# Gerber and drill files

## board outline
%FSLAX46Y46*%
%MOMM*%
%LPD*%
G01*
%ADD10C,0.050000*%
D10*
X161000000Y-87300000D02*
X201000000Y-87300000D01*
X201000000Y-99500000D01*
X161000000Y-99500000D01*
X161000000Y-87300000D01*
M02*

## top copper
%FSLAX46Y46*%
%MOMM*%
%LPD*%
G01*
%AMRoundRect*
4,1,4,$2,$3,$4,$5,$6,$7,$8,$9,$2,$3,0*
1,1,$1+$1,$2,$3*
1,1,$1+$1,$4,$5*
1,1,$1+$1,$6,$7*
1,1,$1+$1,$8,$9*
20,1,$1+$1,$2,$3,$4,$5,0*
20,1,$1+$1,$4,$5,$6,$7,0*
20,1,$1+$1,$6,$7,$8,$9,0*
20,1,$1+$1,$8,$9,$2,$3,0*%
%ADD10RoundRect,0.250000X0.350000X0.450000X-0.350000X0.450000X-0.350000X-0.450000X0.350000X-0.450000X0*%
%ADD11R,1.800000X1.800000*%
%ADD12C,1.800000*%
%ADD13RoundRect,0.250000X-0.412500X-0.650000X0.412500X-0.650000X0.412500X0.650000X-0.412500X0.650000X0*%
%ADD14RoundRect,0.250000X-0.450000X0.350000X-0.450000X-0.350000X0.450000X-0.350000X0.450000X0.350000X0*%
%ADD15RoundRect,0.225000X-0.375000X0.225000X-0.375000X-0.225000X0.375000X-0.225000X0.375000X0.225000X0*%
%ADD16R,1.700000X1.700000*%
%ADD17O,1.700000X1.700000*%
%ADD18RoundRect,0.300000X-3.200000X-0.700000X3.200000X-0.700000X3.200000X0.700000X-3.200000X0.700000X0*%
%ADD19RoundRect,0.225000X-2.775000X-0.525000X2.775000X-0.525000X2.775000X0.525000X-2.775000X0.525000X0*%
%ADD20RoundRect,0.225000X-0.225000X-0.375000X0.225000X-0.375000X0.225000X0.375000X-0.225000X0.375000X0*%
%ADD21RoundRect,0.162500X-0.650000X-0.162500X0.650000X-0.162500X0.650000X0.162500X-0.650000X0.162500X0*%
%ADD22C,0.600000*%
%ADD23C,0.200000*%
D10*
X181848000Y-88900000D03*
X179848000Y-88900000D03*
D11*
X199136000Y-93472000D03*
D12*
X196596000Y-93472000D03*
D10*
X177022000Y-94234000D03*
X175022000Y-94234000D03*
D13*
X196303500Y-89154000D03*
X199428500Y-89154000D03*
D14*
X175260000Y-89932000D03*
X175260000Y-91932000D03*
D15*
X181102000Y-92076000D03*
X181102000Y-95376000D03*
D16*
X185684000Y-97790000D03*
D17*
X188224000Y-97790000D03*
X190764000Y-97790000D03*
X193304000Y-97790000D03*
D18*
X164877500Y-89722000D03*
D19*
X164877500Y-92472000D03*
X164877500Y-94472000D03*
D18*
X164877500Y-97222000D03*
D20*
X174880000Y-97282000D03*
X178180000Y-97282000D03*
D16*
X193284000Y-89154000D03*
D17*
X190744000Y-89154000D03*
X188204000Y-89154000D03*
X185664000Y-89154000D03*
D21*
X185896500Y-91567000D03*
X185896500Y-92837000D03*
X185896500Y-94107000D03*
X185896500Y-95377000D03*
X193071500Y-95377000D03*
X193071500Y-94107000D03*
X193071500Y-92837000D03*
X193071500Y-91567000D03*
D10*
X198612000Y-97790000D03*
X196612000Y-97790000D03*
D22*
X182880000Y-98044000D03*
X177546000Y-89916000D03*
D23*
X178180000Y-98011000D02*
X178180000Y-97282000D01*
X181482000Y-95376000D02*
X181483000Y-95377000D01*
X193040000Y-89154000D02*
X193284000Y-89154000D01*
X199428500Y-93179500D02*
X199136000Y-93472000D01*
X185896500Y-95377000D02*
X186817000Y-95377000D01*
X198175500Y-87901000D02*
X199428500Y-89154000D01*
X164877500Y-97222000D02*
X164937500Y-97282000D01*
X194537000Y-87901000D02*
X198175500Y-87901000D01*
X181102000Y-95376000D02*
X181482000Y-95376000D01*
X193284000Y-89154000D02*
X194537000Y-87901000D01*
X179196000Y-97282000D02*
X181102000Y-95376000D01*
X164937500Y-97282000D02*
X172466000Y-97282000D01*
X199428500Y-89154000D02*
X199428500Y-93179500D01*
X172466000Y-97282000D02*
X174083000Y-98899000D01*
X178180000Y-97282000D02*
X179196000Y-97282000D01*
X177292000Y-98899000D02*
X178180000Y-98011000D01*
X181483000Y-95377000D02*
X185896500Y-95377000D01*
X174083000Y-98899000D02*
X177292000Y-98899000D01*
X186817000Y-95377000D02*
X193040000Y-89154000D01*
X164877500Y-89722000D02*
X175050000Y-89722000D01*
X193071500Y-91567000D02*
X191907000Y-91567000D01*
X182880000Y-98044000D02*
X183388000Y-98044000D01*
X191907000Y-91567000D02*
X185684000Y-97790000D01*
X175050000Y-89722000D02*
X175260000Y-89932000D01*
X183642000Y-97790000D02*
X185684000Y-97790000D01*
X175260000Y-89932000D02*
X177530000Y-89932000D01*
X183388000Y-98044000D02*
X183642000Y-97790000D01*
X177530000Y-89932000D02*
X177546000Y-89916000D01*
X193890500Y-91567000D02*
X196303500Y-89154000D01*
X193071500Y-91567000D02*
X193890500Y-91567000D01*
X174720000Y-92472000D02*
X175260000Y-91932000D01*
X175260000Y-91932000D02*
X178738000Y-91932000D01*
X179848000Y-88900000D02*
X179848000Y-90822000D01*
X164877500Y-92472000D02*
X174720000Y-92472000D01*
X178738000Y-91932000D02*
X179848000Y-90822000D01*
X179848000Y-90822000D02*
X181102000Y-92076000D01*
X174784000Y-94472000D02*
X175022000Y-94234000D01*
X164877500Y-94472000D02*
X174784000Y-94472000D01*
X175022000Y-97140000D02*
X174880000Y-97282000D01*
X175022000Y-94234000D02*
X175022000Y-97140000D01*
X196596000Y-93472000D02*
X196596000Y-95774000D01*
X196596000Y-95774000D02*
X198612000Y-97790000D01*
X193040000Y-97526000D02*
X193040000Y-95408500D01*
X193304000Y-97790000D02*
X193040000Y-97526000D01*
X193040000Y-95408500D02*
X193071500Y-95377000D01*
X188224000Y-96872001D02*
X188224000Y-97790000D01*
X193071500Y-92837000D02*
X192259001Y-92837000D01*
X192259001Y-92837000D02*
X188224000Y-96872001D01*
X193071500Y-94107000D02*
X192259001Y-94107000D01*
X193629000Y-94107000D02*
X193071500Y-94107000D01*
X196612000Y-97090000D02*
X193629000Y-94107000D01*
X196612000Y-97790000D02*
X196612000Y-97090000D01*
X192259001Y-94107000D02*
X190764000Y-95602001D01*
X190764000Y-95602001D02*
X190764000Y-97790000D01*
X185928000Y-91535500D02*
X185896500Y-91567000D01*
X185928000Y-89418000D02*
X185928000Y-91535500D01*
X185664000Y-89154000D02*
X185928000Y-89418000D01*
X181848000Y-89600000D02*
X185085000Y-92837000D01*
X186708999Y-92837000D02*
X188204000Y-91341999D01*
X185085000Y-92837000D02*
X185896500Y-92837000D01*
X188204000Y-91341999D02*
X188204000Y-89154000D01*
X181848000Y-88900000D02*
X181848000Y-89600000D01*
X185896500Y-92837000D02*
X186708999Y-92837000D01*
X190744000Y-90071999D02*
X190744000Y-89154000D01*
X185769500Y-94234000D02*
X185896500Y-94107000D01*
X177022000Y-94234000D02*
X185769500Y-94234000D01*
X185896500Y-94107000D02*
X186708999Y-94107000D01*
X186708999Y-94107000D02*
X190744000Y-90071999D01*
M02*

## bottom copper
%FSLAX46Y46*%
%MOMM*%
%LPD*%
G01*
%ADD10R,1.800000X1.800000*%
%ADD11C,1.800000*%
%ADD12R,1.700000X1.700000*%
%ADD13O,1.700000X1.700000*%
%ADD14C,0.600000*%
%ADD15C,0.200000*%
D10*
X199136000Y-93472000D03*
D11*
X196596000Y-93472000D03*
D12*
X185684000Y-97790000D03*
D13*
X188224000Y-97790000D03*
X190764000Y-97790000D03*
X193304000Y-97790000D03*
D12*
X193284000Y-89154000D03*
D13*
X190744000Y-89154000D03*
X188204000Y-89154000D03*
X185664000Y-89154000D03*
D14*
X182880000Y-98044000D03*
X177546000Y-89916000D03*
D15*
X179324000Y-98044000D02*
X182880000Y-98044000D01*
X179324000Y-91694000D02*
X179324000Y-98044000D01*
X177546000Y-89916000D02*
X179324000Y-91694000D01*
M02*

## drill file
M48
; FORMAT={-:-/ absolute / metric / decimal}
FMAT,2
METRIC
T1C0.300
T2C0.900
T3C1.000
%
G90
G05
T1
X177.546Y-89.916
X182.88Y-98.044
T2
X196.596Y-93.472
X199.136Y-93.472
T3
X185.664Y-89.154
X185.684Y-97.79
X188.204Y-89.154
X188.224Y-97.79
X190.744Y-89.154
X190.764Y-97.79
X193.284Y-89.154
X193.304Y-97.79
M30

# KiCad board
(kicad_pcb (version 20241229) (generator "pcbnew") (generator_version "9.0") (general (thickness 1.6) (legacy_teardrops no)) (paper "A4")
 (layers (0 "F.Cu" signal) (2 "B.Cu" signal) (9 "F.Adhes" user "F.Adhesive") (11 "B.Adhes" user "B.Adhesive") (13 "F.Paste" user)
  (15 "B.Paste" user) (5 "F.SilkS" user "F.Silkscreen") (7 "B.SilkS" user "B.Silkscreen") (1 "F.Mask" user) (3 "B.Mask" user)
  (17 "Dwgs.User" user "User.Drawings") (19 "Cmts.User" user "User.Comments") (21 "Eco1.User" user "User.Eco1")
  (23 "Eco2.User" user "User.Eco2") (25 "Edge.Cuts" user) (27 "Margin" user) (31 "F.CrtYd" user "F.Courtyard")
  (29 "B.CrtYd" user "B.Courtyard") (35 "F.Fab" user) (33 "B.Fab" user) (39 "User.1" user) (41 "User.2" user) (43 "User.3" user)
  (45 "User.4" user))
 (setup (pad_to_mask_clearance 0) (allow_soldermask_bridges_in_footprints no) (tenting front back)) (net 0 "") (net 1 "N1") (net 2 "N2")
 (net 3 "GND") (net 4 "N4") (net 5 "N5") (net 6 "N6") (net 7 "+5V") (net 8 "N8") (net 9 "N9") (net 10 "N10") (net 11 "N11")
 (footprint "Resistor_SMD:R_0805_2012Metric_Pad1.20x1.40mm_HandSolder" (layer "F.Cu") (at 180.848 88.9 180)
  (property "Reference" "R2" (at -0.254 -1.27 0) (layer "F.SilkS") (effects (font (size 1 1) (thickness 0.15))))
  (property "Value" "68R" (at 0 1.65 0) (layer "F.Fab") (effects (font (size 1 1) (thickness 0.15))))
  (pad "1" smd roundrect (at -1 0 180) (size 1.2 1.4) (layers "F.Cu" "F.Mask" "F.Paste") (roundrect_rratio 0.208333) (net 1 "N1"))
  (pad "2" smd roundrect (at 1 0 180) (size 1.2 1.4) (layers "F.Cu" "F.Mask" "F.Paste") (roundrect_rratio 0.208333) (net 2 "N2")))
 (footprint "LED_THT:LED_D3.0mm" (layer "F.Cu") (at 199.136 93.472 180)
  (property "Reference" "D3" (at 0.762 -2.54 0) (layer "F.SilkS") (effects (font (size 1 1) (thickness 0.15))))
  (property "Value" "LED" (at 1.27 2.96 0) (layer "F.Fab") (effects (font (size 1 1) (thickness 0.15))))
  (pad "1" thru_hole rect (at 0 0 180) (size 1.8 1.8) (drill 0.9) (layers "*.Cu" "*.Mask") (remove_unused_layers no) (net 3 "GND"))
  (pad "2" thru_hole circle (at 2.54 0 180) (size 1.8 1.8) (drill 0.9) (layers "*.Cu" "*.Mask") (remove_unused_layers no) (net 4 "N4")))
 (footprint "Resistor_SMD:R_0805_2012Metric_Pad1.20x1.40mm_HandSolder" (layer "F.Cu") (at 176.022 94.234 180)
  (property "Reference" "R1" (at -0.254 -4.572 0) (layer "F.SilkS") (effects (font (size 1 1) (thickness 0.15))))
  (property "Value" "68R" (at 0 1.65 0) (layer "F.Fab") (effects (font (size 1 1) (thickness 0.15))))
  (pad "1" smd roundrect (at -1 0 180) (size 1.2 1.4) (layers "F.Cu" "F.Mask" "F.Paste") (roundrect_rratio 0.208333) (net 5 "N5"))
  (pad "2" smd roundrect (at 1 0 180) (size 1.2 1.4) (layers "F.Cu" "F.Mask" "F.Paste") (roundrect_rratio 0.208333) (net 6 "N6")))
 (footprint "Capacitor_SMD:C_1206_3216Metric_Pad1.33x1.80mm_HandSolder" (layer "F.Cu") (at 197.866 89.154)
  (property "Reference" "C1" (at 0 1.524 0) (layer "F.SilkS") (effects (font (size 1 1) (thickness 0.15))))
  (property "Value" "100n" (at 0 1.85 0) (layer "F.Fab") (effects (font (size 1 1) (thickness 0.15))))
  (pad "1" smd roundrect (at -1.5625 0) (size 1.325 1.8) (layers "F.Cu" "F.Mask" "F.Paste") (roundrect_rratio 0.188679) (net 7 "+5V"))
  (pad "2" smd roundrect (at 1.5625 0) (size 1.325 1.8) (layers "F.Cu" "F.Mask" "F.Paste") (roundrect_rratio 0.188679) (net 3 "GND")))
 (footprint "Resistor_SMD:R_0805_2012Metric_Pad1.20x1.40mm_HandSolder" (layer "F.Cu") (at 175.26 90.932 -90)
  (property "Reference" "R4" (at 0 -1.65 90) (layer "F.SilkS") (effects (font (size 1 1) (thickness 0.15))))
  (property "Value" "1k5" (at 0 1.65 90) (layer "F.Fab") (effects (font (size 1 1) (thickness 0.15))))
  (pad "1" smd roundrect (at -1 0 270) (size 1.2 1.4) (layers "F.Cu" "F.Mask" "F.Paste") (roundrect_rratio 0.208333) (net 7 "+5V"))
  (pad "2" smd roundrect (at 1 0 270) (size 1.2 1.4) (layers "F.Cu" "F.Mask" "F.Paste") (roundrect_rratio 0.208333) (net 2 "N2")))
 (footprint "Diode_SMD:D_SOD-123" (layer "F.Cu") (at 181.102 93.726 -90)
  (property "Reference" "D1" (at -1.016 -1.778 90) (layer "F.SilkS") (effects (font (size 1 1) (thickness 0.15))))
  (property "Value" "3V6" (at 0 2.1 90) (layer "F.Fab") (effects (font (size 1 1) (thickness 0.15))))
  (pad "1" smd roundrect (at -1.65 0 270) (size 0.9 1.2) (layers "F.Cu" "F.Mask" "F.Paste") (roundrect_rratio 0.25) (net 2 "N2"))
  (pad "2" smd roundrect (at 1.65 0 270) (size 0.9 1.2) (layers "F.Cu" "F.Mask" "F.Paste") (roundrect_rratio 0.25) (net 3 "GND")))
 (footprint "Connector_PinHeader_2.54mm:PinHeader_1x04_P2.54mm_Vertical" (layer "F.Cu") (at 185.684 97.79 90)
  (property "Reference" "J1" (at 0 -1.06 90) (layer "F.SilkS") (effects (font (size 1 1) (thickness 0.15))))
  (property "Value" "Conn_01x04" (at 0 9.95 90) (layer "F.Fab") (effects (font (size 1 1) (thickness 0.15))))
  (pad "1" thru_hole rect (at 0 0 90) (size 1.7 1.7) (drill 1) (layers "*.Cu" "*.Mask") (remove_unused_layers no) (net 7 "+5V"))
  (pad "2" thru_hole oval (at 0 2.54 90) (size 1.7 1.7) (drill 1) (layers "*.Cu" "*.Mask") (remove_unused_layers no) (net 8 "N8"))
  (pad "3" thru_hole oval (at 0 5.08 90) (size 1.7 1.7) (drill 1) (layers "*.Cu" "*.Mask") (remove_unused_layers no) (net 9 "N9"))
  (pad "4" thru_hole oval (at 0 7.62 90) (size 1.7 1.7) (drill 1) (layers "*.Cu" "*.Mask") (remove_unused_layers no) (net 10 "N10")))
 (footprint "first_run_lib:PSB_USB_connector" (layer "F.Cu") (at 164.8775 93.472)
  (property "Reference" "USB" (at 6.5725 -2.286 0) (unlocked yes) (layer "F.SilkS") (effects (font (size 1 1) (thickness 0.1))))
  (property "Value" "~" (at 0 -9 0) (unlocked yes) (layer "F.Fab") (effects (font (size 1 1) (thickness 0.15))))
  (pad "1" smd roundrect (at 0 -3.75) (size 7 2) (layers "F.Cu" "F.Mask" "F.Paste") (roundrect_rratio 0.15) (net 7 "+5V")
   (thermal_bridge_angle 45))
  (pad "2" smd roundrect (at 0 -1) (size 6 1.5) (layers "F.Cu" "F.Mask" "F.Paste") (roundrect_rratio 0.15) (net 2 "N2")
   (thermal_bridge_angle 45))
  (pad "3" smd roundrect (at 0 1) (size 6 1.5) (layers "F.Cu" "F.Mask" "F.Paste") (roundrect_rratio 0.15) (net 6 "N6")
   (thermal_bridge_angle 45))
  (pad "4" smd roundrect (at 0 3.75) (size 7 2) (layers "F.Cu" "F.Mask" "F.Paste") (roundrect_rratio 0.15) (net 3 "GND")
   (thermal_bridge_angle 45)))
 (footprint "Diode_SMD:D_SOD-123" (layer "F.Cu") (at 176.53 97.282)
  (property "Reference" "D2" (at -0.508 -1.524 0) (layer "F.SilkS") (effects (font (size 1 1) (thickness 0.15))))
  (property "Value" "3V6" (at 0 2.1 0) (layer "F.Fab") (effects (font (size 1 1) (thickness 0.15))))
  (pad "1" smd roundrect (at -1.65 0) (size 0.9 1.2) (layers "F.Cu" "F.Mask" "F.Paste") (roundrect_rratio 0.25) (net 6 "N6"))
  (pad "2" smd roundrect (at 1.65 0) (size 0.9 1.2) (layers "F.Cu" "F.Mask" "F.Paste") (roundrect_rratio 0.25) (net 3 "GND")))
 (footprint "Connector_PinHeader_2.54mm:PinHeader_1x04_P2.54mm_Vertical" (layer "F.Cu") (at 193.284 89.154 -90)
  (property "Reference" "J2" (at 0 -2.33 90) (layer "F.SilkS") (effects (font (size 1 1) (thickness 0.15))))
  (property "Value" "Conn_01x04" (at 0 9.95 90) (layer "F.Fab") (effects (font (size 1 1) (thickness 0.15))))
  (pad "1" thru_hole rect (at 0 0 270) (size 1.7 1.7) (drill 1) (layers "*.Cu" "*.Mask") (remove_unused_layers no) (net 3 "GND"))
  (pad "2" thru_hole oval (at 0 2.54 270) (size 1.7 1.7) (drill 1) (layers "*.Cu" "*.Mask") (remove_unused_layers no) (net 5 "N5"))
  (pad "3" thru_hole oval (at 0 5.08 270) (size 1.7 1.7) (drill 1) (layers "*.Cu" "*.Mask") (remove_unused_layers no) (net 1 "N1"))
  (pad "4" thru_hole oval (at 0 7.62 270) (size 1.7 1.7) (drill 1) (layers "*.Cu" "*.Mask") (remove_unused_layers no) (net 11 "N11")))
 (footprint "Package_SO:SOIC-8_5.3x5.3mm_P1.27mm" (layer "F.Cu") (at 189.484 93.472)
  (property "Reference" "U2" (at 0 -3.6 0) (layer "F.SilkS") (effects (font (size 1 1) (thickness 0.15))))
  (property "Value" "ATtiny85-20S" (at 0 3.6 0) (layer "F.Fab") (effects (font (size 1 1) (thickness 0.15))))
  (pad "1" smd roundrect (at -3.5875 -1.905) (size 1.625 0.65) (layers "F.Cu" "F.Mask" "F.Paste") (roundrect_rratio 0.25) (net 11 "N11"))
  (pad "2" smd roundrect (at -3.5875 -0.635) (size 1.625 0.65) (layers "F.Cu" "F.Mask" "F.Paste") (roundrect_rratio 0.25) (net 1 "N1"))
  (pad "3" smd roundrect (at -3.5875 0.635) (size 1.625 0.65) (layers "F.Cu" "F.Mask" "F.Paste") (roundrect_rratio 0.25) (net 5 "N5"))
  (pad "4" smd roundrect (at -3.5875 1.905) (size 1.625 0.65) (layers "F.Cu" "F.Mask" "F.Paste") (roundrect_rratio 0.25) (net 3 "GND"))
  (pad "5" smd roundrect (at 3.5875 1.905) (size 1.625 0.65) (layers "F.Cu" "F.Mask" "F.Paste") (roundrect_rratio 0.25) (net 10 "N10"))
  (pad "6" smd roundrect (at 3.5875 0.635) (size 1.625 0.65) (layers "F.Cu" "F.Mask" "F.Paste") (roundrect_rratio 0.25) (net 9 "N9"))
  (pad "7" smd roundrect (at 3.5875 -0.635) (size 1.625 0.65) (layers "F.Cu" "F.Mask" "F.Paste") (roundrect_rratio 0.25) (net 8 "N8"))
  (pad "8" smd roundrect (at 3.5875 -1.905) (size 1.625 0.65) (layers "F.Cu" "F.Mask" "F.Paste") (roundrect_rratio 0.25) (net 7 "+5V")))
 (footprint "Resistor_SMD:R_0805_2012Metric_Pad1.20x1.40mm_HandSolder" (layer "F.Cu") (at 197.612 97.79 180)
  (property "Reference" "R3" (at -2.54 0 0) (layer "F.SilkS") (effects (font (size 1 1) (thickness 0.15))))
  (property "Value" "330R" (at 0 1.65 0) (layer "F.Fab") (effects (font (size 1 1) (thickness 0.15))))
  (pad "1" smd roundrect (at -1 0 180) (size 1.2 1.4) (layers "F.Cu" "F.Mask" "F.Paste") (roundrect_rratio 0.208333) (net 4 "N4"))
  (pad "2" smd roundrect (at 1 0 180) (size 1.2 1.4) (layers "F.Cu" "F.Mask" "F.Paste") (roundrect_rratio 0.208333) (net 9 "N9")))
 (gr_rect (start 161 87.3) (end 201 99.5) (stroke (width 0.05) (type solid)) (fill no) (layer "Edge.Cuts"))
 (segment (start 178.18 98.011) (end 178.18 97.282) (width 0.2) (layer "F.Cu") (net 3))
 (segment (start 181.482 95.376) (end 181.483 95.377) (width 0.2) (layer "F.Cu") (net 3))
 (segment (start 193.04 89.154) (end 193.284 89.154) (width 0.2) (layer "F.Cu") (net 3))
 (segment (start 199.4285 93.1795) (end 199.136 93.472) (width 0.2) (layer "F.Cu") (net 3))
 (segment (start 185.8965 95.377) (end 186.817 95.377) (width 0.2) (layer "F.Cu") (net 3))
 (segment (start 198.1755 87.901) (end 199.4285 89.154) (width 0.2) (layer "F.Cu") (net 3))
 (segment (start 164.8775 97.222) (end 164.9375 97.282) (width 0.2) (layer "F.Cu") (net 3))
 (segment (start 194.537 87.901) (end 198.1755 87.901) (width 0.2) (layer "F.Cu") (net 3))
 (segment (start 181.102 95.376) (end 181.482 95.376) (width 0.2) (layer "F.Cu") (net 3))
 (segment (start 193.284 89.154) (end 194.537 87.901) (width 0.2) (layer "F.Cu") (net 3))
 (segment (start 179.196 97.282) (end 181.102 95.376) (width 0.2) (layer "F.Cu") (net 3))
 (segment (start 164.9375 97.282) (end 172.466 97.282) (width 0.2) (layer "F.Cu") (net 3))
 (segment (start 199.4285 89.154) (end 199.4285 93.1795) (width 0.2) (layer "F.Cu") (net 3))
 (segment (start 172.466 97.282) (end 174.083 98.899) (width 0.2) (layer "F.Cu") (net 3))
 (segment (start 178.18 97.282) (end 179.196 97.282) (width 0.2) (layer "F.Cu") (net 3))
 (segment (start 177.292 98.899) (end 178.18 98.011) (width 0.2) (layer "F.Cu") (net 3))
 (segment (start 181.483 95.377) (end 185.8965 95.377) (width 0.2) (layer "F.Cu") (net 3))
 (segment (start 174.083 98.899) (end 177.292 98.899) (width 0.2) (layer "F.Cu") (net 3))
 (segment (start 186.817 95.377) (end 193.04 89.154) (width 0.2) (layer "F.Cu") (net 3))
 (segment (start 164.8775 89.722) (end 175.05 89.722) (width 0.2) (layer "F.Cu") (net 7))
 (segment (start 193.0715 91.567) (end 191.907 91.567) (width 0.2) (layer "F.Cu") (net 7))
 (segment (start 182.88 98.044) (end 183.388 98.044) (width 0.2) (layer "F.Cu") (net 7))
 (segment (start 191.907 91.567) (end 185.684 97.79) (width 0.2) (layer "F.Cu") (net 7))
 (segment (start 175.05 89.722) (end 175.26 89.932) (width 0.2) (layer "F.Cu") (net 7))
 (segment (start 183.642 97.79) (end 185.684 97.79) (width 0.2) (layer "F.Cu") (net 7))
 (segment (start 175.26 89.932) (end 177.53 89.932) (width 0.2) (layer "F.Cu") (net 7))
 (segment (start 183.388 98.044) (end 183.642 97.79) (width 0.2) (layer "F.Cu") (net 7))
 (segment (start 177.53 89.932) (end 177.546 89.916) (width 0.2) (layer "F.Cu") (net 7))
 (segment (start 193.8905 91.567) (end 196.3035 89.154) (width 0.2) (layer "F.Cu") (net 7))
 (segment (start 193.0715 91.567) (end 193.8905 91.567) (width 0.2) (layer "F.Cu") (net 7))
 (via (at 182.88 98.044) (size 0.6) (drill 0.3) (layers "F.Cu" "B.Cu") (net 7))
 (via (at 177.546 89.916) (size 0.6) (drill 0.3) (layers "F.Cu" "B.Cu") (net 7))
 (segment (start 179.324 98.044) (end 182.88 98.044) (width 0.2) (layer "B.Cu") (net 7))
 (segment (start 179.324 91.694) (end 179.324 98.044) (width 0.2) (layer "B.Cu") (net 7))
 (segment (start 177.546 89.916) (end 179.324 91.694) (width 0.2) (layer "B.Cu") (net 7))
 (segment (start 174.72 92.472) (end 175.26 91.932) (width 0.2) (layer "F.Cu") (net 2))
 (segment (start 175.26 91.932) (end 178.738 91.932) (width 0.2) (layer "F.Cu") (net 2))
 (segment (start 179.848 88.9) (end 179.848 90.822) (width 0.2) (layer "F.Cu") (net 2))
 (segment (start 164.8775 92.472) (end 174.72 92.472) (width 0.2) (layer "F.Cu") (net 2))
 (segment (start 178.738 91.932) (end 179.848 90.822) (width 0.2) (layer "F.Cu") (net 2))
 (segment (start 179.848 90.822) (end 181.102 92.076) (width 0.2) (layer "F.Cu") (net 2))
 (segment (start 174.784 94.472) (end 175.022 94.234) (width 0.2) (layer "F.Cu") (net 6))
 (segment (start 164.8775 94.472) (end 174.784 94.472) (width 0.2) (layer "F.Cu") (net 6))
 (segment (start 175.022 97.14) (end 174.88 97.282) (width 0.2) (layer "F.Cu") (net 6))
 (segment (start 175.022 94.234) (end 175.022 97.14) (width 0.2) (layer "F.Cu") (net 6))
 (segment (start 196.596 93.472) (end 196.596 95.774) (width 0.2) (layer "F.Cu") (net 4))
 (segment (start 196.596 95.774) (end 198.612 97.79) (width 0.2) (layer "F.Cu") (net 4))
 (segment (start 193.04 97.526) (end 193.04 95.4085) (width 0.2) (layer "F.Cu") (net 10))
 (segment (start 193.304 97.79) (end 193.04 97.526) (width 0.2) (layer "F.Cu") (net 10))
 (segment (start 193.04 95.4085) (end 193.0715 95.377) (width 0.2) (layer "F.Cu") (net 10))
 (segment (start 188.224 96.872001) (end 188.224 97.79) (width 0.2) (layer "F.Cu") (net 8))
 (segment (start 193.0715 92.837) (end 192.259001 92.837) (width 0.2) (layer "F.Cu") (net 8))
 (segment (start 192.259001 92.837) (end 188.224 96.872001) (width 0.2) (layer "F.Cu") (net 8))
 (segment (start 193.0715 94.107) (end 192.259001 94.107) (width 0.2) (layer "F.Cu") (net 9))
 (segment (start 193.629 94.107) (end 193.0715 94.107) (width 0.2) (layer "F.Cu") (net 9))
 (segment (start 196.612 97.09) (end 193.629 94.107) (width 0.2) (layer "F.Cu") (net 9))
 (segment (start 196.612 97.79) (end 196.612 97.09) (width 0.2) (layer "F.Cu") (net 9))
 (segment (start 192.259001 94.107) (end 190.764 95.602001) (width 0.2) (layer "F.Cu") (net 9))
 (segment (start 190.764 95.602001) (end 190.764 97.79) (width 0.2) (layer "F.Cu") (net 9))
 (segment (start 185.928 91.5355) (end 185.8965 91.567) (width 0.2) (layer "F.Cu") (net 11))
 (segment (start 185.928 89.418) (end 185.928 91.5355) (width 0.2) (layer "F.Cu") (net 11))
 (segment (start 185.664 89.154) (end 185.928 89.418) (width 0.2) (layer "F.Cu") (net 11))
 (segment (start 181.848 89.6) (end 185.085 92.837) (width 0.2) (layer "F.Cu") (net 1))
 (segment (start 186.708999 92.837) (end 188.204 91.341999) (width 0.2) (layer "F.Cu") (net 1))
 (segment (start 185.085 92.837) (end 185.8965 92.837) (width 0.2) (layer "F.Cu") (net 1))
 (segment (start 188.204 91.341999) (end 188.204 89.154) (width 0.2) (layer "F.Cu") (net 1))
 (segment (start 181.848 88.9) (end 181.848 89.6) (width 0.2) (layer "F.Cu") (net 1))
 (segment (start 185.8965 92.837) (end 186.708999 92.837) (width 0.2) (layer "F.Cu") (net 1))
 (segment (start 190.744 90.071999) (end 190.744 89.154) (width 0.2) (layer "F.Cu") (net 5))
 (segment (start 185.7695 94.234) (end 185.8965 94.107) (width 0.2) (layer "F.Cu") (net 5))
 (segment (start 177.022 94.234) (end 185.7695 94.234) (width 0.2) (layer "F.Cu") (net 5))
 (segment (start 185.8965 94.107) (end 186.708999 94.107) (width 0.2) (layer "F.Cu") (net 5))
 (segment (start 186.708999 94.107) (end 190.744 90.071999) (width 0.2) (layer "F.Cu") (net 5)))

